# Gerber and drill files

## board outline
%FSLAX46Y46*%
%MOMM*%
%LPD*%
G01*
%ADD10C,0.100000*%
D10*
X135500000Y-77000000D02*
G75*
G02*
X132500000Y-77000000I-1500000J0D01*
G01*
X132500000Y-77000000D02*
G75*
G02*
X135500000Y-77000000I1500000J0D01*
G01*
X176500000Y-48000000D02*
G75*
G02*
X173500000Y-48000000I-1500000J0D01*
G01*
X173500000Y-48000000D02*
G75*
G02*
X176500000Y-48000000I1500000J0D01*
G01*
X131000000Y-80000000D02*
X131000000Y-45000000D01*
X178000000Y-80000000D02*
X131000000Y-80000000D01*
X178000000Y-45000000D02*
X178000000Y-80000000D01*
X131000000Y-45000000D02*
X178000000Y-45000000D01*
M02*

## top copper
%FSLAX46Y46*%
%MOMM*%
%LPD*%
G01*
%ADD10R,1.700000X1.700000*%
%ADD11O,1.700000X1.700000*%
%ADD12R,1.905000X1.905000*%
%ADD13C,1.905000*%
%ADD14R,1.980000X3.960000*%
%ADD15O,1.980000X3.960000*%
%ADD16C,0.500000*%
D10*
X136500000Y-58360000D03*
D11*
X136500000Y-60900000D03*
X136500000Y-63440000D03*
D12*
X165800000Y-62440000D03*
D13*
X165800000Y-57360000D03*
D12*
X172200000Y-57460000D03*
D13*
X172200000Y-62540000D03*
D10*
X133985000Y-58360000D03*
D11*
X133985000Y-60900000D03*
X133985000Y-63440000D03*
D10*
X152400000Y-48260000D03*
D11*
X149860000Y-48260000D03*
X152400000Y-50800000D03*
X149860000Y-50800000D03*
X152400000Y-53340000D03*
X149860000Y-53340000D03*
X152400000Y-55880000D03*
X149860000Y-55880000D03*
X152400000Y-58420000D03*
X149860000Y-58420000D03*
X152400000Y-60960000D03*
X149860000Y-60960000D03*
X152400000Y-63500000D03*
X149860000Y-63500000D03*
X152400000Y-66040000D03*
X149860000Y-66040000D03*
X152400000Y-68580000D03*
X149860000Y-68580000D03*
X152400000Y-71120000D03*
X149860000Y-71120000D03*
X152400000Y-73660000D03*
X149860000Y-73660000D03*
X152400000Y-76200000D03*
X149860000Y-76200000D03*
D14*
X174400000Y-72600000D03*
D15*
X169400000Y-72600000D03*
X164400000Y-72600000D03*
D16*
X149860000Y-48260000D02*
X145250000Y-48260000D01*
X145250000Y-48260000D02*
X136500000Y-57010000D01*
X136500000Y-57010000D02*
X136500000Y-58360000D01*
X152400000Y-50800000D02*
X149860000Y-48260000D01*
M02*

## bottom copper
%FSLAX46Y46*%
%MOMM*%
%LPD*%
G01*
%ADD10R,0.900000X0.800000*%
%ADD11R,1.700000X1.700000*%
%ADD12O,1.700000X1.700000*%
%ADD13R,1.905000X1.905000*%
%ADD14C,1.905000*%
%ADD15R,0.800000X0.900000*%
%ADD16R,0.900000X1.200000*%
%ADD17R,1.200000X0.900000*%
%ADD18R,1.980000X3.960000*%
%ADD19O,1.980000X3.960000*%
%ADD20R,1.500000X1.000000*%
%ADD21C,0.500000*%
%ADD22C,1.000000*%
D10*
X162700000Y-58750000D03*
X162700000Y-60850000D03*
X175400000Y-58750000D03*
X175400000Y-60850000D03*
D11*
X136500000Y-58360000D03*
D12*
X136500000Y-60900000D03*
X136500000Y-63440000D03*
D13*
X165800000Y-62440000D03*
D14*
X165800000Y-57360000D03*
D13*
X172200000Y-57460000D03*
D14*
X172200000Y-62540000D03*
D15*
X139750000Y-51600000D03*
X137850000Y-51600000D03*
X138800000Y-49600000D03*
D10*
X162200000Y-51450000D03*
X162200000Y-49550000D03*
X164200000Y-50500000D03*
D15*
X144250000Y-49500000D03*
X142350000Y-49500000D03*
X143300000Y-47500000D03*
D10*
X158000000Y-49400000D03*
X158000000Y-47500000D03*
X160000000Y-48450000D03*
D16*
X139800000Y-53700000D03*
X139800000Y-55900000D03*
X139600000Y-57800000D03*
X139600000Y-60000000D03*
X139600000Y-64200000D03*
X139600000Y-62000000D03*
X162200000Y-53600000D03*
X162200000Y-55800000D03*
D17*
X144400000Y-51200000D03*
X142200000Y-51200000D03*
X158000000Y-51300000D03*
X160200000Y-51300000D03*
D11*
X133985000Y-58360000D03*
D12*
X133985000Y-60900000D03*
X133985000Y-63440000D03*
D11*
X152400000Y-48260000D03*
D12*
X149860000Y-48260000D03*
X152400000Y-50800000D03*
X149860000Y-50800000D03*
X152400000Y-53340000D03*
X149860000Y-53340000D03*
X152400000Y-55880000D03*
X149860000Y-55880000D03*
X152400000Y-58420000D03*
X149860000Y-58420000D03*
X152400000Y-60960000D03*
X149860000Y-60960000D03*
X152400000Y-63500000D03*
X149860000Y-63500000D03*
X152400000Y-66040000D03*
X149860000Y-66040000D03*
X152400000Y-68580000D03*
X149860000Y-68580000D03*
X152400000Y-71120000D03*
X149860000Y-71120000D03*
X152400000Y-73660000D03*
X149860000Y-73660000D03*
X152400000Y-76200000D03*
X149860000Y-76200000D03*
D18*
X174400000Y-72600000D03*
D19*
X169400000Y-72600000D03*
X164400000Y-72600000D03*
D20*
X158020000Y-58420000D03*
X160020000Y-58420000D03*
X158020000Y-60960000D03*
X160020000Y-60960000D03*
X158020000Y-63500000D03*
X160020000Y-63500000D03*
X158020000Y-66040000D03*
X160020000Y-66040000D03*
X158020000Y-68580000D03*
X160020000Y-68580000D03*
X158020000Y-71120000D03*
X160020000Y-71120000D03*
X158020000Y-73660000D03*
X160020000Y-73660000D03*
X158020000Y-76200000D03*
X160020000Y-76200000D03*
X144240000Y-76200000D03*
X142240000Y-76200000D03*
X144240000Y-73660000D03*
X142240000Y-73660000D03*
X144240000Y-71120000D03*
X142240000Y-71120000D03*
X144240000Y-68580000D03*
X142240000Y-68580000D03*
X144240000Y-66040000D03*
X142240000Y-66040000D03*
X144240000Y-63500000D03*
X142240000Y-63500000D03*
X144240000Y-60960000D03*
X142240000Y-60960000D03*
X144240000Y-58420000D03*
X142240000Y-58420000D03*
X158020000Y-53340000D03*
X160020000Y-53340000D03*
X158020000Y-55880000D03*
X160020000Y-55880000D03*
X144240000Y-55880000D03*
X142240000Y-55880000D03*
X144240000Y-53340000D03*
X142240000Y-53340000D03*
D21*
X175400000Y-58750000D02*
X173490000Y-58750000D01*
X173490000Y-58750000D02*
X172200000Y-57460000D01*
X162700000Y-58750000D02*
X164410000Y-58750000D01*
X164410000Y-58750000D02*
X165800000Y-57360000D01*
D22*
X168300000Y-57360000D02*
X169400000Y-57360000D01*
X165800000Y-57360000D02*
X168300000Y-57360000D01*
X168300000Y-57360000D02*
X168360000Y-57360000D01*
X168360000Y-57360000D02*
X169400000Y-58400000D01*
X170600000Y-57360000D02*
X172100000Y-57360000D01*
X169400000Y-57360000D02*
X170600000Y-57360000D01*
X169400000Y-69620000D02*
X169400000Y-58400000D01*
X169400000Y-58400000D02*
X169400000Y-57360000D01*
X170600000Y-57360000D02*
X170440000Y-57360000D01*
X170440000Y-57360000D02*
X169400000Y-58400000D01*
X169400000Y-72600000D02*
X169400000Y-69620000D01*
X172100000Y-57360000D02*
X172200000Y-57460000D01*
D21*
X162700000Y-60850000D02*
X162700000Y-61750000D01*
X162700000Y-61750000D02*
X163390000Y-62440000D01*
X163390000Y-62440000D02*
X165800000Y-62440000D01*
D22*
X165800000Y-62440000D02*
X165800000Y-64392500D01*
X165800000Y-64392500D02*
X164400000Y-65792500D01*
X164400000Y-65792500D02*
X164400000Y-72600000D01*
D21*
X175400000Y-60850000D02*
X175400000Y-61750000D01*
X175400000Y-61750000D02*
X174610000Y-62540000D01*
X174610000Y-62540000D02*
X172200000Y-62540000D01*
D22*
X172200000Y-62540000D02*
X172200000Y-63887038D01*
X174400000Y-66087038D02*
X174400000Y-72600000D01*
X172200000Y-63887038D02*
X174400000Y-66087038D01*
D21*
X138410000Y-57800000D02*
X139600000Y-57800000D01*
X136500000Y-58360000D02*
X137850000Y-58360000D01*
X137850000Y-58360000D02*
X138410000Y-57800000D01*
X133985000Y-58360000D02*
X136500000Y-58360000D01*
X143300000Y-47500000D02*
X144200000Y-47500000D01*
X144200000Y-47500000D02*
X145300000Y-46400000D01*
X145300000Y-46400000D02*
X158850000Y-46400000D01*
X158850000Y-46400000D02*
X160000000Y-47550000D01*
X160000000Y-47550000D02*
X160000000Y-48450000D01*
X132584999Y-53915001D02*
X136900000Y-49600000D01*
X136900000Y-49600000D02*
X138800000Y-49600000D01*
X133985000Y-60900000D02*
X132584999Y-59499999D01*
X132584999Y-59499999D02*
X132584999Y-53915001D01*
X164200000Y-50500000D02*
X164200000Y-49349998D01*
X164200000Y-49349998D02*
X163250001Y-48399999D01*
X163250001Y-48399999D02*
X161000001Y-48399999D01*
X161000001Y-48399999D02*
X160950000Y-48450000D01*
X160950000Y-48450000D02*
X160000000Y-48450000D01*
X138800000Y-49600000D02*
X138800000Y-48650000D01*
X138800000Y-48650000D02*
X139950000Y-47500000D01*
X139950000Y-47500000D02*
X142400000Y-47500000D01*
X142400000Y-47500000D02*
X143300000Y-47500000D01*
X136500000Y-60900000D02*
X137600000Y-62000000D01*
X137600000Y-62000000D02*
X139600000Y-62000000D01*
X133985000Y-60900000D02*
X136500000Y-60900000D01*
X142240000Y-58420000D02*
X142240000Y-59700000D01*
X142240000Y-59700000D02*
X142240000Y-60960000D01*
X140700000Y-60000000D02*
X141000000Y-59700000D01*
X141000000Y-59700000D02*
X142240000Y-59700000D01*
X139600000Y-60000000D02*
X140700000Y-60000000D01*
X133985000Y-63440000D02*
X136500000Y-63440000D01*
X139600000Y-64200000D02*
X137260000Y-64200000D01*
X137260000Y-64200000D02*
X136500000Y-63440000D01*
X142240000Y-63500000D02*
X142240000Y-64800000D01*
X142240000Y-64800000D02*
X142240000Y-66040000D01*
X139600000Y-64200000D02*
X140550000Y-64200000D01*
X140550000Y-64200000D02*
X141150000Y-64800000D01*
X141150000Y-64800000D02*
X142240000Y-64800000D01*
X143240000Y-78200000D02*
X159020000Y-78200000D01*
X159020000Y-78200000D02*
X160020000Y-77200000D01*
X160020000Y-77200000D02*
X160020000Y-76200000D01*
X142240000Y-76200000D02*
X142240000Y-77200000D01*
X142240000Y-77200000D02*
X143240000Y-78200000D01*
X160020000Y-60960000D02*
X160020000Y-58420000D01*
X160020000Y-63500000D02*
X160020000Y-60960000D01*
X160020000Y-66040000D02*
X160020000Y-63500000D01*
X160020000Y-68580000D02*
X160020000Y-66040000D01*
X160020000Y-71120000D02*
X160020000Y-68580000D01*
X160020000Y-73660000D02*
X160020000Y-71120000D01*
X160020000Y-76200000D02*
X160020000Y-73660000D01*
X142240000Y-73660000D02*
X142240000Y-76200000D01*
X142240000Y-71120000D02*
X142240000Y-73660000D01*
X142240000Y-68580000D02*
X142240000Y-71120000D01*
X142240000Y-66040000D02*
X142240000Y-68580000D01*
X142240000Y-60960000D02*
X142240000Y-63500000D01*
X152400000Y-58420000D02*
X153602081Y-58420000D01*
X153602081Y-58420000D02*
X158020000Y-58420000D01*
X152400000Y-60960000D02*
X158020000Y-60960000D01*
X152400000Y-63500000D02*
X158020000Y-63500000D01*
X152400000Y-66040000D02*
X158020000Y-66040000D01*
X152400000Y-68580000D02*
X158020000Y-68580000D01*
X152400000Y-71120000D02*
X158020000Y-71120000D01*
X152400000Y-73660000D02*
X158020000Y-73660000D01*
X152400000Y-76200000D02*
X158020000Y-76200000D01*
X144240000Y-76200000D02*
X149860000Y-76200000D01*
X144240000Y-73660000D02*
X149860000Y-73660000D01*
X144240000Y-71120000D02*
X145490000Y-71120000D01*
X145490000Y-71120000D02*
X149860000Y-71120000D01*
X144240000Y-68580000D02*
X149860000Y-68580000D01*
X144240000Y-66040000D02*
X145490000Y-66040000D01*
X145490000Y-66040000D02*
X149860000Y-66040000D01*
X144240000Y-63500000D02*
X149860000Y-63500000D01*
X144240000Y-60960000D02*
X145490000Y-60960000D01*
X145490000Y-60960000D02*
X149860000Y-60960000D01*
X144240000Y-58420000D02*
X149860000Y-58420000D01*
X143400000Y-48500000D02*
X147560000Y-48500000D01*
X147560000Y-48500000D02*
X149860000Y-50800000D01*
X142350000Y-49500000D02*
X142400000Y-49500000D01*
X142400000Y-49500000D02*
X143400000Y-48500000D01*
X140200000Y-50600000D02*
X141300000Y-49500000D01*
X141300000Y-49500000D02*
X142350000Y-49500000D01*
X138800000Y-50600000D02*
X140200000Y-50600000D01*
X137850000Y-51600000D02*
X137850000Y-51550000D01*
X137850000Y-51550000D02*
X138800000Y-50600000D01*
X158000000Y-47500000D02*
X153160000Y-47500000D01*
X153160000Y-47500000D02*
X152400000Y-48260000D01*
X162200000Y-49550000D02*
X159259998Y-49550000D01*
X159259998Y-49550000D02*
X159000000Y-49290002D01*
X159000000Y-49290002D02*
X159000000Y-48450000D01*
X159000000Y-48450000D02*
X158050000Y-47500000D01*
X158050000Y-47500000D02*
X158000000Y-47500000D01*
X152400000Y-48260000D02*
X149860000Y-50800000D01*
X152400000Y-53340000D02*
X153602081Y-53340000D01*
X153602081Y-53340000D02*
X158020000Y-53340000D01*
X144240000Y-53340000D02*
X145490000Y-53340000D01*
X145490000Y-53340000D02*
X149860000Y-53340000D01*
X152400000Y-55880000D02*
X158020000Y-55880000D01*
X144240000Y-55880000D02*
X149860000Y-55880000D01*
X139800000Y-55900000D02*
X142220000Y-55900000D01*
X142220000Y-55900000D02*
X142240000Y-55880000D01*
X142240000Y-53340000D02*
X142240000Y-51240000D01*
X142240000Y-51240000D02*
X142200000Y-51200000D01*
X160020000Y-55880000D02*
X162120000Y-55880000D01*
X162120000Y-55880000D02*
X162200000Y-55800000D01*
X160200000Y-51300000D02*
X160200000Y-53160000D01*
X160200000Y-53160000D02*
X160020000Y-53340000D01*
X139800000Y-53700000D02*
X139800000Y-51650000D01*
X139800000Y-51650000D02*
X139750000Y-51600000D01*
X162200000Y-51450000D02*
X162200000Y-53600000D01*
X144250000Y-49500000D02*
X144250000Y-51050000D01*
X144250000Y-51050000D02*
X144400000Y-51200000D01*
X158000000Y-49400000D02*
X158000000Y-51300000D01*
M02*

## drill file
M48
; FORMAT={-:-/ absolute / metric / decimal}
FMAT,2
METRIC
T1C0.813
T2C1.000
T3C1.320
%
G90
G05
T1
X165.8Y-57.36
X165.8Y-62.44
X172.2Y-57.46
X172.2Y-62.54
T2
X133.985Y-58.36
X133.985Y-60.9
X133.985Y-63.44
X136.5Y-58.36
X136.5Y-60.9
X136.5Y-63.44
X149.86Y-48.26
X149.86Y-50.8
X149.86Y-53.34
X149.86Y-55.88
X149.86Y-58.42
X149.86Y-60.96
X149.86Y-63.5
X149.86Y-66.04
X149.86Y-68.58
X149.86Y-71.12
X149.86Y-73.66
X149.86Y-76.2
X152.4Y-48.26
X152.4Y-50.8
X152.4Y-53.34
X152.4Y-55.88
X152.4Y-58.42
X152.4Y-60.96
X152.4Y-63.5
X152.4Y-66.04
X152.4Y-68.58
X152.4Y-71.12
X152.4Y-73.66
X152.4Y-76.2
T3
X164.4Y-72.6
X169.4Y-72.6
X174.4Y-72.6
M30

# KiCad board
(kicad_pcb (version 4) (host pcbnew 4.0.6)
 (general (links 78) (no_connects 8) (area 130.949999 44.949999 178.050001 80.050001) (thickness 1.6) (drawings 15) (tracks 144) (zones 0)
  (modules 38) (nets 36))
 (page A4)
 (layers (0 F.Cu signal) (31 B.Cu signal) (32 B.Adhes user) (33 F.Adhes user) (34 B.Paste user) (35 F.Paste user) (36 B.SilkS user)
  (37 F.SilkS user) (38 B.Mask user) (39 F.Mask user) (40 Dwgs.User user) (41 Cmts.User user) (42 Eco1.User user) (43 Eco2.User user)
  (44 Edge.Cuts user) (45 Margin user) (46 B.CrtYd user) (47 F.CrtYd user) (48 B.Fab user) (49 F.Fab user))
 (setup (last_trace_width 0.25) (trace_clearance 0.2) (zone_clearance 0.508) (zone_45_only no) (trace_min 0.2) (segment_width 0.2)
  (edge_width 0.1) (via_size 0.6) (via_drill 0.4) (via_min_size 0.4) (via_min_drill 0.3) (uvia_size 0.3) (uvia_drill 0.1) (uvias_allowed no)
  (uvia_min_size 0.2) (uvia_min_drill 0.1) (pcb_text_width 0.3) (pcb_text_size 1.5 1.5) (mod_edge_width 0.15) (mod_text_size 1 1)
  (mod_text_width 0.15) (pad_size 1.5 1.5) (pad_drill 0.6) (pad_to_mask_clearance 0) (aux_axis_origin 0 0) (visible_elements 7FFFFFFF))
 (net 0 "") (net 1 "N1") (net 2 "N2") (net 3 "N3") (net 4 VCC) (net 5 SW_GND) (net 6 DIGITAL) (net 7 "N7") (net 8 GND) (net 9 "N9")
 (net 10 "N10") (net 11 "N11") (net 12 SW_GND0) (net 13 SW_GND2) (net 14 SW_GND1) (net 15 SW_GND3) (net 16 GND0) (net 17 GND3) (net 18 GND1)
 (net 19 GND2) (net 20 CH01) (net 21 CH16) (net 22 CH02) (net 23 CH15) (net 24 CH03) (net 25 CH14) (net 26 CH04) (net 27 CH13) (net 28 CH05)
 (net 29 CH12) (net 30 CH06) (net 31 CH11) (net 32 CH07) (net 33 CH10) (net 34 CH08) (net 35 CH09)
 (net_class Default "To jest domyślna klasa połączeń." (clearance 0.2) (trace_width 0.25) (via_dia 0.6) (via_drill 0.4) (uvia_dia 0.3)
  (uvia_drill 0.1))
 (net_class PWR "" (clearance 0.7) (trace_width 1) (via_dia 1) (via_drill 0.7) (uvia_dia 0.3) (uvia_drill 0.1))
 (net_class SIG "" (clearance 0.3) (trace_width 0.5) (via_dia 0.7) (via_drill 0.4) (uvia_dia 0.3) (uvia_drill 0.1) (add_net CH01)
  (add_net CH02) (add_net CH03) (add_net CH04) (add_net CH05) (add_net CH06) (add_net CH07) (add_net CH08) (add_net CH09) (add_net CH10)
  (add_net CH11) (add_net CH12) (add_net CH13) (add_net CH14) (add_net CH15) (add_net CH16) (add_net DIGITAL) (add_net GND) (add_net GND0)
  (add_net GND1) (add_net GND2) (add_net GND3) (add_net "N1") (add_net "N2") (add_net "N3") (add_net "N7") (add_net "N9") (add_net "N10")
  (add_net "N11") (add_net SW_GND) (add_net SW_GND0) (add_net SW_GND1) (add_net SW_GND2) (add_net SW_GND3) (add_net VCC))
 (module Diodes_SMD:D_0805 (layer B.Cu) (at 162.7 59.8 270)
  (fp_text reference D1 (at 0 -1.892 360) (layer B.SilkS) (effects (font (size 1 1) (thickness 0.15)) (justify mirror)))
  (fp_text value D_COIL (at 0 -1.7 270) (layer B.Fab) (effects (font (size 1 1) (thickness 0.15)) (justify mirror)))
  (pad 1 smd rect (at -1.05 0 270) (size 0.8 0.9) (layers B.Cu B.Paste B.Mask) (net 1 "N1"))
  (pad 2 smd rect (at 1.05 0 270) (size 0.8 0.9) (layers B.Cu B.Paste B.Mask) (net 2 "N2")))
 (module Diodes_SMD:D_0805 (layer B.Cu) (at 175.4 59.8 270)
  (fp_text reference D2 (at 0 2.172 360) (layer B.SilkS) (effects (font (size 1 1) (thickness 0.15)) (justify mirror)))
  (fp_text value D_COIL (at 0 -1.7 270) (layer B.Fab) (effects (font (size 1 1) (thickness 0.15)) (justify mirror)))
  (pad 1 smd rect (at -1.05 0 270) (size 0.8 0.9) (layers B.Cu B.Paste B.Mask) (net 1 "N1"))
  (pad 2 smd rect (at 1.05 0 270) (size 0.8 0.9) (layers B.Cu B.Paste B.Mask) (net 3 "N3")))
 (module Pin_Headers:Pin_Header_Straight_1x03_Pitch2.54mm (layer F.Cu) (at 136.5 58.36)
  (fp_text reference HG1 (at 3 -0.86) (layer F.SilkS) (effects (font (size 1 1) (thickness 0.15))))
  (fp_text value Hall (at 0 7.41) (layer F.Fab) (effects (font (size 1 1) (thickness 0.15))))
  (pad 1 thru_hole rect (at 0 0) (size 1.7 1.7) (drill 1) (layers *.Cu *.Mask) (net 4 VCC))
  (pad 2 thru_hole oval (at 0 2.54) (size 1.7 1.7) (drill 1) (layers *.Cu *.Mask) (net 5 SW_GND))
  (pad 3 thru_hole oval (at 0 5.08) (size 1.7 1.7) (drill 1) (layers *.Cu *.Mask) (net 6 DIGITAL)))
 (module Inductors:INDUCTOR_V (layer F.Cu) (at 165.8 59.9 90)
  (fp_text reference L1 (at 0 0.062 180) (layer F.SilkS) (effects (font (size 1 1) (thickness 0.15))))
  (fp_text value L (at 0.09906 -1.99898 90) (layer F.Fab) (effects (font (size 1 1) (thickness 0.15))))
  (pad 1 thru_hole rect (at -2.54 0 90) (size 1.905 1.905) (drill 0.8128) (layers *.Cu *.Mask) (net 2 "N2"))
  (pad 2 thru_hole circle (at 2.54 0 90) (size 1.905 1.905) (drill 0.8128) (layers *.Cu *.Mask) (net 1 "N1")))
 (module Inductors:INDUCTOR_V (layer F.Cu) (at 172.2 60 270)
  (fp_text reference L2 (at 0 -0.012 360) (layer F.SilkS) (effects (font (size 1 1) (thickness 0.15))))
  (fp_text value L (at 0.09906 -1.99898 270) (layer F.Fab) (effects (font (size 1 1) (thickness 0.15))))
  (pad 1 thru_hole rect (at -2.54 0 270) (size 1.905 1.905) (drill 0.8128) (layers *.Cu *.Mask) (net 1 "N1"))
  (pad 2 thru_hole circle (at 2.54 0 270) (size 1.905 1.905) (drill 0.8128) (layers *.Cu *.Mask) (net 3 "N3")))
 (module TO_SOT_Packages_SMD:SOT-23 (layer B.Cu) (at 138.8 50.6 90)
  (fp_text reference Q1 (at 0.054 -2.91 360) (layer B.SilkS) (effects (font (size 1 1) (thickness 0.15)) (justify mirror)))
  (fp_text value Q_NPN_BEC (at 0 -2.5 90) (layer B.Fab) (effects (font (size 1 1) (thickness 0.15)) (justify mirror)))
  (pad 1 smd rect (at -1 0.95 90) (size 0.9 0.8) (layers B.Cu B.Paste B.Mask) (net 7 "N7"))
  (pad 2 smd rect (at -1 -0.95 90) (size 0.9 0.8) (layers B.Cu B.Paste B.Mask) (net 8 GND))
  (pad 3 smd rect (at 1 0 90) (size 0.9 0.8) (layers B.Cu B.Paste B.Mask) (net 5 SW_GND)))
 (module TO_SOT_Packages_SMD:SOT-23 (layer B.Cu) (at 163.2 50.5)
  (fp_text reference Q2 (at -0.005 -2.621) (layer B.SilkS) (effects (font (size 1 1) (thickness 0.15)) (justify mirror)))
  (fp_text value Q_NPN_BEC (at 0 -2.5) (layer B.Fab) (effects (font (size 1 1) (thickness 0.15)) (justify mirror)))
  (pad 1 smd rect (at -1 0.95) (size 0.9 0.8) (layers B.Cu B.Paste B.Mask) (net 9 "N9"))
  (pad 2 smd rect (at -1 -0.95) (size 0.9 0.8) (layers B.Cu B.Paste B.Mask) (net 8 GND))
  (pad 3 smd rect (at 1 0) (size 0.9 0.8) (layers B.Cu B.Paste B.Mask) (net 5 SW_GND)))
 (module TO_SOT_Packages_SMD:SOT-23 (layer B.Cu) (at 143.3 48.5 90)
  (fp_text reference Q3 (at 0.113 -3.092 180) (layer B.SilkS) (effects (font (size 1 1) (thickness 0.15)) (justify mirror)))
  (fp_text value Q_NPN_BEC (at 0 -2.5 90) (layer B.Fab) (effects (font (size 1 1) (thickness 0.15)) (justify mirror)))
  (pad 1 smd rect (at -1 0.95 90) (size 0.9 0.8) (layers B.Cu B.Paste B.Mask) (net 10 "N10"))
  (pad 2 smd rect (at -1 -0.95 90) (size 0.9 0.8) (layers B.Cu B.Paste B.Mask) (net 8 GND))
  (pad 3 smd rect (at 1 0 90) (size 0.9 0.8) (layers B.Cu B.Paste B.Mask) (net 5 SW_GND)))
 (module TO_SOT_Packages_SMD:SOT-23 (layer B.Cu) (at 159 48.45)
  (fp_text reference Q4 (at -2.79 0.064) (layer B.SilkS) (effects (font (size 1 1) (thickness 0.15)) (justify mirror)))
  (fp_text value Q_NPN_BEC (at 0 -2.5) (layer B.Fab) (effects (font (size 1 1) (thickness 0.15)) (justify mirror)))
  (pad 1 smd rect (at -1 0.95) (size 0.9 0.8) (layers B.Cu B.Paste B.Mask) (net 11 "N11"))
  (pad 2 smd rect (at -1 -0.95) (size 0.9 0.8) (layers B.Cu B.Paste B.Mask) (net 8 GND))
  (pad 3 smd rect (at 1 0) (size 0.9 0.8) (layers B.Cu B.Paste B.Mask) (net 5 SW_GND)))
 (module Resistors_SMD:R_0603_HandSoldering (layer B.Cu) (at 139.8 54.8 270)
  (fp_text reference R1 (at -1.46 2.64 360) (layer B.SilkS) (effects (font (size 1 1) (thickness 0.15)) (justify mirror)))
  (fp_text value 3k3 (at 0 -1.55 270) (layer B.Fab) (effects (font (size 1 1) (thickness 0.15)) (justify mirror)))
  (pad 1 smd rect (at -1.1 0 270) (size 1.2 0.9) (layers B.Cu B.Paste B.Mask) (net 7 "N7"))
  (pad 2 smd rect (at 1.1 0 270) (size 1.2 0.9) (layers B.Cu B.Paste B.Mask) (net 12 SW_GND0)))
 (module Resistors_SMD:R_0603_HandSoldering (layer B.Cu) (at 139.6 58.9 270)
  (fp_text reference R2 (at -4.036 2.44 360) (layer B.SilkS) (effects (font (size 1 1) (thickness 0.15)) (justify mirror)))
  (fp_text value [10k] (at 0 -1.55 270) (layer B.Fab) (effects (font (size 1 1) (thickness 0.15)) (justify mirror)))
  (pad 1 smd rect (at -1.1 0 270) (size 1.2 0.9) (layers B.Cu B.Paste B.Mask) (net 4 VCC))
  (pad 2 smd rect (at 1.1 0 270) (size 1.2 0.9) (layers B.Cu B.Paste B.Mask) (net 6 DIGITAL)))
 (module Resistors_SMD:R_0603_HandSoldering (layer B.Cu) (at 139.6 63.1 90)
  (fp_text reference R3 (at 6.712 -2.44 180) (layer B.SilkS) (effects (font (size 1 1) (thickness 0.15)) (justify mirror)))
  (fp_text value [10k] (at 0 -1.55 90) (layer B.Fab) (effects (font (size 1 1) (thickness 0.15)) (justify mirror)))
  (pad 1 smd rect (at -1.1 0 90) (size 1.2 0.9) (layers B.Cu B.Paste B.Mask) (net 6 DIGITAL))
  (pad 2 smd rect (at 1.1 0 90) (size 1.2 0.9) (layers B.Cu B.Paste B.Mask) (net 5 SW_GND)))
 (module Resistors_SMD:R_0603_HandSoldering (layer B.Cu) (at 162.2 54.7 270)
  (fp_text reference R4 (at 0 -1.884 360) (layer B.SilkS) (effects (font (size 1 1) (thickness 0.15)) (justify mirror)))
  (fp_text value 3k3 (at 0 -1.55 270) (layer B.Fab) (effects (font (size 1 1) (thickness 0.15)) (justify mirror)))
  (pad 1 smd rect (at -1.1 0 270) (size 1.2 0.9) (layers B.Cu B.Paste B.Mask) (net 9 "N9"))
  (pad 2 smd rect (at 1.1 0 270) (size 1.2 0.9) (layers B.Cu B.Paste B.Mask) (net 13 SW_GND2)))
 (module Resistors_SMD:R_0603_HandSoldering (layer B.Cu) (at 143.3 51.2 180)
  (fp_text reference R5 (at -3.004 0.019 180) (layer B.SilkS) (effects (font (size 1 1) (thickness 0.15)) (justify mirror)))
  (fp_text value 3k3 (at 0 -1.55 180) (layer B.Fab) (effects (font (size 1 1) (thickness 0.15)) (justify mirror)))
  (pad 1 smd rect (at -1.1 0 180) (size 1.2 0.9) (layers B.Cu B.Paste B.Mask) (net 10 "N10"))
  (pad 2 smd rect (at 1.1 0 180) (size 1.2 0.9) (layers B.Cu B.Paste B.Mask) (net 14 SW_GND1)))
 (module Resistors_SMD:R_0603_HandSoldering (layer B.Cu) (at 159.1 51.3)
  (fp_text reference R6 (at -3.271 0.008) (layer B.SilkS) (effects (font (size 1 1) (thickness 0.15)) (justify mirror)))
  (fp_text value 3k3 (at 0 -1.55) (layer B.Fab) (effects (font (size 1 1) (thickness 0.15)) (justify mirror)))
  (pad 1 smd rect (at -1.1 0) (size 1.2 0.9) (layers B.Cu B.Paste B.Mask) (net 11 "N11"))
  (pad 2 smd rect (at 1.1 0) (size 1.2 0.9) (layers B.Cu B.Paste B.Mask) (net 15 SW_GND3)))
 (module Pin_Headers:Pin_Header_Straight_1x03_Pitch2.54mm (layer F.Cu) (at 133.985 58.36)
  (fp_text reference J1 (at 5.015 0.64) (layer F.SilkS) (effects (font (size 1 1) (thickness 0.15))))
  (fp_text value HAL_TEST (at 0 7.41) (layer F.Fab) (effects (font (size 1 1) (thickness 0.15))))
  (pad 1 thru_hole rect (at 0 0) (size 1.7 1.7) (drill 1) (layers *.Cu *.Mask) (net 4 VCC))
  (pad 2 thru_hole oval (at 0 2.54) (size 1.7 1.7) (drill 1) (layers *.Cu *.Mask) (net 5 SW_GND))
  (pad 3 thru_hole oval (at 0 5.08) (size 1.7 1.7) (drill 1) (layers *.Cu *.Mask) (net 6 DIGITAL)))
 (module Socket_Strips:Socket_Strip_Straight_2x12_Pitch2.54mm (layer F.Cu) (at 152.4 48.26)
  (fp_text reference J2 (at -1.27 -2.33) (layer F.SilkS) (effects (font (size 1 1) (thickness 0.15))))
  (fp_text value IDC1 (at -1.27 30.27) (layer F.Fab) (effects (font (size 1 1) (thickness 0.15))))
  (pad 1 thru_hole rect (at 0 0) (size 1.7 1.7) (drill 1) (layers *.Cu *.Mask) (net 8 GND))
  (pad 2 thru_hole oval (at -2.54 0) (size 1.7 1.7) (drill 1) (layers *.Cu *.Mask) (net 4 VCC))
  (pad 3 thru_hole oval (at 0 2.54) (size 1.7 1.7) (drill 1) (layers *.Cu *.Mask) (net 4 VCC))
  (pad 4 thru_hole oval (at -2.54 2.54) (size 1.7 1.7) (drill 1) (layers *.Cu *.Mask) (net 8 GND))
  (pad 5 thru_hole oval (at 0 5.08) (size 1.7 1.7) (drill 1) (layers *.Cu *.Mask) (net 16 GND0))
  (pad 6 thru_hole oval (at -2.54 5.08) (size 1.7 1.7) (drill 1) (layers *.Cu *.Mask) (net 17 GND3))
  (pad 7 thru_hole oval (at 0 7.62) (size 1.7 1.7) (drill 1) (layers *.Cu *.Mask) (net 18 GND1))
  (pad 8 thru_hole oval (at -2.54 7.62) (size 1.7 1.7) (drill 1) (layers *.Cu *.Mask) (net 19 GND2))
  (pad 9 thru_hole oval (at 0 10.16) (size 1.7 1.7) (drill 1) (layers *.Cu *.Mask) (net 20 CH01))
  (pad 10 thru_hole oval (at -2.54 10.16) (size 1.7 1.7) (drill 1) (layers *.Cu *.Mask) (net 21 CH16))
  (pad 11 thru_hole oval (at 0 12.7) (size 1.7 1.7) (drill 1) (layers *.Cu *.Mask) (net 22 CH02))
  (pad 12 thru_hole oval (at -2.54 12.7) (size 1.7 1.7) (drill 1) (layers *.Cu *.Mask) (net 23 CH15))
  (pad 13 thru_hole oval (at 0 15.24) (size 1.7 1.7) (drill 1) (layers *.Cu *.Mask) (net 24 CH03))
  (pad 14 thru_hole oval (at -2.54 15.24) (size 1.7 1.7) (drill 1) (layers *.Cu *.Mask) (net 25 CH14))
  (pad 15 thru_hole oval (at 0 17.78) (size 1.7 1.7) (drill 1) (layers *.Cu *.Mask) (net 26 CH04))
  (pad 16 thru_hole oval (at -2.54 17.78) (size 1.7 1.7) (drill 1) (layers *.Cu *.Mask) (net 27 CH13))
  (pad 17 thru_hole oval (at 0 20.32) (size 1.7 1.7) (drill 1) (layers *.Cu *.Mask) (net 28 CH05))
  (pad 18 thru_hole oval (at -2.54 20.32) (size 1.7 1.7) (drill 1) (layers *.Cu *.Mask) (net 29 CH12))
  (pad 19 thru_hole oval (at 0 22.86) (size 1.7 1.7) (drill 1) (layers *.Cu *.Mask) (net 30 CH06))
  (pad 20 thru_hole oval (at -2.54 22.86) (size 1.7 1.7) (drill 1) (layers *.Cu *.Mask) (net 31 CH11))
  (pad 21 thru_hole oval (at 0 25.4) (size 1.7 1.7) (drill 1) (layers *.Cu *.Mask) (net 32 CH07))
  (pad 22 thru_hole oval (at -2.54 25.4) (size 1.7 1.7) (drill 1) (layers *.Cu *.Mask) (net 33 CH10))
  (pad 23 thru_hole oval (at 0 27.94) (size 1.7 1.7) (drill 1) (layers *.Cu *.Mask) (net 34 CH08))
  (pad 24 thru_hole oval (at -2.54 27.94) (size 1.7 1.7) (drill 1) (layers *.Cu *.Mask) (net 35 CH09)))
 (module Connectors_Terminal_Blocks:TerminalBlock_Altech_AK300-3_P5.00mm (layer F.Cu) (at 174.4 72.6 180)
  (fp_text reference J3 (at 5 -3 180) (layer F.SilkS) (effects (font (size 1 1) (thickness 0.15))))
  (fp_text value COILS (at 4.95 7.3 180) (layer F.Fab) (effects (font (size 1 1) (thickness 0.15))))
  (pad 1 thru_hole rect (at 0 0 180) (size 1.98 3.96) (drill 1.32) (layers *.Cu *.Mask) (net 3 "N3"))
  (pad 2 thru_hole oval (at 5 0 180) (size 1.98 3.96) (drill 1.32) (layers *.Cu *.Mask) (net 1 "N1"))
  (pad 3 thru_hole oval (at 10 0 180) (size 1.98 3.96) (drill 1.32) (layers *.Cu *.Mask) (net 2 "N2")))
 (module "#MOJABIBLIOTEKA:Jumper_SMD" (layer B.Cu) (at 159.02 58.42)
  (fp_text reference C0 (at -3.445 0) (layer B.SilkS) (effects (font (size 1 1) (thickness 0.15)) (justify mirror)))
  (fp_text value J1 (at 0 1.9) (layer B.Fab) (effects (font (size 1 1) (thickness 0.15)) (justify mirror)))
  (pad 1 smd rect (at -1 0) (size 1.5 1) (layers B.Cu B.Paste B.Mask) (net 20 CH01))
  (pad 2 smd rect (at 1 0) (size 1.5 1) (layers B.Cu B.Paste B.Mask) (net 6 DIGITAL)))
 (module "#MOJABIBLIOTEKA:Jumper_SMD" (layer B.Cu) (at 159.02 60.96)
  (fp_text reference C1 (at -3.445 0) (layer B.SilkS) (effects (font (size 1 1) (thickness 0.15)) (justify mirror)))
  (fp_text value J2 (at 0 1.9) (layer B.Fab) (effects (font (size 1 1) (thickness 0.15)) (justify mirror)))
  (pad 1 smd rect (at -1 0) (size 1.5 1) (layers B.Cu B.Paste B.Mask) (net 22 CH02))
  (pad 2 smd rect (at 1 0) (size 1.5 1) (layers B.Cu B.Paste B.Mask) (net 6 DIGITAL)))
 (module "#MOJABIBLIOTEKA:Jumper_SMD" (layer B.Cu) (at 159.02 63.5)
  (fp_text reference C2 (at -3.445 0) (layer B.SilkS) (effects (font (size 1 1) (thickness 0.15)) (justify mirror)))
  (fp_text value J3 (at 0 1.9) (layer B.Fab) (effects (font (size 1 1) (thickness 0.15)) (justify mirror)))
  (pad 1 smd rect (at -1 0) (size 1.5 1) (layers B.Cu B.Paste B.Mask) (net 24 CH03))
  (pad 2 smd rect (at 1 0) (size 1.5 1) (layers B.Cu B.Paste B.Mask) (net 6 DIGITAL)))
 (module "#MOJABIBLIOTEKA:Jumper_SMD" (layer B.Cu) (at 159.02 66.04)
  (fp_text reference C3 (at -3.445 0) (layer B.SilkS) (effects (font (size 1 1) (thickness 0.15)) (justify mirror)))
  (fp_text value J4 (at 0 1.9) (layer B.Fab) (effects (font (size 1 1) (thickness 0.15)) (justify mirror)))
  (pad 1 smd rect (at -1 0) (size 1.5 1) (layers B.Cu B.Paste B.Mask) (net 26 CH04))
  (pad 2 smd rect (at 1 0) (size 1.5 1) (layers B.Cu B.Paste B.Mask) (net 6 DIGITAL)))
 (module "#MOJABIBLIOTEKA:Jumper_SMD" (layer B.Cu) (at 159.02 68.58)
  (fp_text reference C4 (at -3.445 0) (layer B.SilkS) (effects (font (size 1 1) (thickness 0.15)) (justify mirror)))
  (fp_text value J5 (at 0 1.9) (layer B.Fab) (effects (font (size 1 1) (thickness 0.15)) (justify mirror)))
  (pad 1 smd rect (at -1 0) (size 1.5 1) (layers B.Cu B.Paste B.Mask) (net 28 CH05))
  (pad 2 smd rect (at 1 0) (size 1.5 1) (layers B.Cu B.Paste B.Mask) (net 6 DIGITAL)))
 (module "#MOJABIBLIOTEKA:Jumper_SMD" (layer B.Cu) (at 159.02 71.12)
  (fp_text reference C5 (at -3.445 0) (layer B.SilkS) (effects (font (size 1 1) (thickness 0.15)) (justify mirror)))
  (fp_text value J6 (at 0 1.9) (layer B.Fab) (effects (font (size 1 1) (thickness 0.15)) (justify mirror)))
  (pad 1 smd rect (at -1 0) (size 1.5 1) (layers B.Cu B.Paste B.Mask) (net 30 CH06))
  (pad 2 smd rect (at 1 0) (size 1.5 1) (layers B.Cu B.Paste B.Mask) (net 6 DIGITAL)))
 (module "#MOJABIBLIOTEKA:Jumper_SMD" (layer B.Cu) (at 159.02 73.66)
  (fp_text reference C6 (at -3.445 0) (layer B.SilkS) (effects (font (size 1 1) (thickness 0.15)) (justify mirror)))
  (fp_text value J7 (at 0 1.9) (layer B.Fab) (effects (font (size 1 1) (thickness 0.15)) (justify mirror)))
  (pad 1 smd rect (at -1 0) (size 1.5 1) (layers B.Cu B.Paste B.Mask) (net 32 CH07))
  (pad 2 smd rect (at 1 0) (size 1.5 1) (layers B.Cu B.Paste B.Mask) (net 6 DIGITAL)))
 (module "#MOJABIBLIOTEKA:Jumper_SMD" (layer B.Cu) (at 159.02 76.2)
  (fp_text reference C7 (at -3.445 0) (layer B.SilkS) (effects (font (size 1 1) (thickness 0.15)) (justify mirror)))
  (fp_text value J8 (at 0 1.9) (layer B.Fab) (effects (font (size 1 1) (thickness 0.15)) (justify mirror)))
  (pad 1 smd rect (at -1 0) (size 1.5 1) (layers B.Cu B.Paste B.Mask) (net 34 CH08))
  (pad 2 smd rect (at 1 0) (size 1.5 1) (layers B.Cu B.Paste B.Mask) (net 6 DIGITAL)))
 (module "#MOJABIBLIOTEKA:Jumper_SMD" (layer B.Cu) (at 143.24 76.2 180)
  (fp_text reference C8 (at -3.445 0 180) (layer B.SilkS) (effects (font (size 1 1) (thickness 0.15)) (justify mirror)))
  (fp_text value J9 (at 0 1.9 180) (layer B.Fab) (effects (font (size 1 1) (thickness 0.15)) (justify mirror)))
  (pad 1 smd rect (at -1 0 180) (size 1.5 1) (layers B.Cu B.Paste B.Mask) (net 35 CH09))
  (pad 2 smd rect (at 1 0 180) (size 1.5 1) (layers B.Cu B.Paste B.Mask) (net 6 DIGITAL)))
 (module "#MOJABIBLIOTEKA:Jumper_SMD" (layer B.Cu) (at 143.24 73.66 180)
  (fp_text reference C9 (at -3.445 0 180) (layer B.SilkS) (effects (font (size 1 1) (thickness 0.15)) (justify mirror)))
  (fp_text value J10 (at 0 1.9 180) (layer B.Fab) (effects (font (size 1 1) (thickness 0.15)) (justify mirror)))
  (pad 1 smd rect (at -1 0 180) (size 1.5 1) (layers B.Cu B.Paste B.Mask) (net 33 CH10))
  (pad 2 smd rect (at 1 0 180) (size 1.5 1) (layers B.Cu B.Paste B.Mask) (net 6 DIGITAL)))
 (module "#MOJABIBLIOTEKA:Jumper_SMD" (layer B.Cu) (at 143.24 71.12 180)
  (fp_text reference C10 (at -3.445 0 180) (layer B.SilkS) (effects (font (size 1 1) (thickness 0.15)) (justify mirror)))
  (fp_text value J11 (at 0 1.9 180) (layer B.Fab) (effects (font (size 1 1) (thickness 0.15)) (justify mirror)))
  (pad 1 smd rect (at -1 0 180) (size 1.5 1) (layers B.Cu B.Paste B.Mask) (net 31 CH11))
  (pad 2 smd rect (at 1 0 180) (size 1.5 1) (layers B.Cu B.Paste B.Mask) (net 6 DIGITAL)))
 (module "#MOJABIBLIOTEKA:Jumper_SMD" (layer B.Cu) (at 143.24 68.58 180)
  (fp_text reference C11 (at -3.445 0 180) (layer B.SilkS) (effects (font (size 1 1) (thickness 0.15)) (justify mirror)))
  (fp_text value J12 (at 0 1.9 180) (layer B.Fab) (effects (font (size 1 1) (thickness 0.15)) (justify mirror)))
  (pad 1 smd rect (at -1 0 180) (size 1.5 1) (layers B.Cu B.Paste B.Mask) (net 29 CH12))
  (pad 2 smd rect (at 1 0 180) (size 1.5 1) (layers B.Cu B.Paste B.Mask) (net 6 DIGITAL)))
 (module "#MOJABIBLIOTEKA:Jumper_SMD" (layer B.Cu) (at 143.24 66.04 180)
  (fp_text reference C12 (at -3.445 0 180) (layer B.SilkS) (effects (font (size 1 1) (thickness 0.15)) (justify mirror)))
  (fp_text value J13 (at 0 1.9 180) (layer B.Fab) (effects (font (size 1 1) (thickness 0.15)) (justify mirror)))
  (pad 1 smd rect (at -1 0 180) (size 1.5 1) (layers B.Cu B.Paste B.Mask) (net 27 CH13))
  (pad 2 smd rect (at 1 0 180) (size 1.5 1) (layers B.Cu B.Paste B.Mask) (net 6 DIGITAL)))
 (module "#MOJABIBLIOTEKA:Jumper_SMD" (layer B.Cu) (at 143.24 63.5 180)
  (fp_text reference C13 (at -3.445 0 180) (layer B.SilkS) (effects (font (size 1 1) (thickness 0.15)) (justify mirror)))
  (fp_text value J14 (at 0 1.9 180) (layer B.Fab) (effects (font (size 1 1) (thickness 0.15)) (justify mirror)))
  (pad 1 smd rect (at -1 0 180) (size 1.5 1) (layers B.Cu B.Paste B.Mask) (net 25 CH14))
  (pad 2 smd rect (at 1 0 180) (size 1.5 1) (layers B.Cu B.Paste B.Mask) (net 6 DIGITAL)))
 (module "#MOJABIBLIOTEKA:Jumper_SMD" (layer B.Cu) (at 143.24 60.96 180)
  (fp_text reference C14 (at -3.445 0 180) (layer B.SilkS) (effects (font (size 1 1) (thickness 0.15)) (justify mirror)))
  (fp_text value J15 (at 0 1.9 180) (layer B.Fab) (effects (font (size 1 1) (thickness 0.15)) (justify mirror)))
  (pad 1 smd rect (at -1 0 180) (size 1.5 1) (layers B.Cu B.Paste B.Mask) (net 23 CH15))
  (pad 2 smd rect (at 1 0 180) (size 1.5 1) (layers B.Cu B.Paste B.Mask) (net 6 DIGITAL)))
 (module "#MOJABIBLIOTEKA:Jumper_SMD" (layer B.Cu) (at 143.24 58.42 180)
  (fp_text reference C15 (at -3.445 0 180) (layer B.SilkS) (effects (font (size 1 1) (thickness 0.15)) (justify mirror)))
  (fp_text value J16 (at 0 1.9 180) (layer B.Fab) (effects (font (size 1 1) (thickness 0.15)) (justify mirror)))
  (pad 1 smd rect (at -1 0 180) (size 1.5 1) (layers B.Cu B.Paste B.Mask) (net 21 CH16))
  (pad 2 smd rect (at 1 0 180) (size 1.5 1) (layers B.Cu B.Paste B.Mask) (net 6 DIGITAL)))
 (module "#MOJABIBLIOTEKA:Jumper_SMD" (layer B.Cu) (at 159.02 53.34)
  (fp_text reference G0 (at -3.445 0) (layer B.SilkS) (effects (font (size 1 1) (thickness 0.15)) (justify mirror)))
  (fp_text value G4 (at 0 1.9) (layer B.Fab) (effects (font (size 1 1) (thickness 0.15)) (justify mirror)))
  (pad 1 smd rect (at -1 0) (size 1.5 1) (layers B.Cu B.Paste B.Mask) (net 16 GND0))
  (pad 2 smd rect (at 1 0) (size 1.5 1) (layers B.Cu B.Paste B.Mask) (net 15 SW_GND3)))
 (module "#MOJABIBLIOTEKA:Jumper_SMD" (layer B.Cu) (at 159.02 55.88)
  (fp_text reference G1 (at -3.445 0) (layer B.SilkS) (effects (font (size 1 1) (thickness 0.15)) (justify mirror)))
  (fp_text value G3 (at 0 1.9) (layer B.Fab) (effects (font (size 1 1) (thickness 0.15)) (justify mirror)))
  (pad 1 smd rect (at -1 0) (size 1.5 1) (layers B.Cu B.Paste B.Mask) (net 18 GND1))
  (pad 2 smd rect (at 1 0) (size 1.5 1) (layers B.Cu B.Paste B.Mask) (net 13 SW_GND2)))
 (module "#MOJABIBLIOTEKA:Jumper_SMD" (layer B.Cu) (at 143.24 55.88 180)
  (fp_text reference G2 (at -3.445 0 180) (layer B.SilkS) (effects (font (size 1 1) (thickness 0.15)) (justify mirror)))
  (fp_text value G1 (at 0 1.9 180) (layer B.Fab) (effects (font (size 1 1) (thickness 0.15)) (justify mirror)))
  (pad 1 smd rect (at -1 0 180) (size 1.5 1) (layers B.Cu B.Paste B.Mask) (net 19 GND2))
  (pad 2 smd rect (at 1 0 180) (size 1.5 1) (layers B.Cu B.Paste B.Mask) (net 12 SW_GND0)))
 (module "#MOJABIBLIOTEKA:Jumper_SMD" (layer B.Cu) (at 143.24 53.34 180)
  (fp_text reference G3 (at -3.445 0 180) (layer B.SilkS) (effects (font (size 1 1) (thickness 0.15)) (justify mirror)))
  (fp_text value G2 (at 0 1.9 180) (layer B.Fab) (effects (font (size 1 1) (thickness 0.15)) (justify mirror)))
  (pad 1 smd rect (at -1 0 180) (size 1.5 1) (layers B.Cu B.Paste B.Mask) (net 17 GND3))
  (pad 2 smd rect (at 1 0 180) (size 1.5 1) (layers B.Cu B.Paste B.Mask) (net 14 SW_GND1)))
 (gr_circle (center 134 77) (end 134 78.5) (layer Edge.Cuts) (width 0.1))
 (gr_circle (center 175 48) (end 175 46.5) (layer Edge.Cuts) (width 0.1))
 (gr_line (start 131 80) (end 131 45) (layer Edge.Cuts) (width 0.1))
 (gr_line (start 178 80) (end 131 80) (layer Edge.Cuts) (width 0.1))
 (gr_line (start 178 45) (end 178 80) (layer Edge.Cuts) (width 0.1))
 (gr_line (start 131 45) (end 178 45) (layer Edge.Cuts) (width 0.1))
 (segment (start 175.4 58.75) (end 173.49 58.75) (width 0.5) (layer B.Cu) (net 1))
 (segment (start 173.49 58.75) (end 172.2 57.46) (width 0.5) (layer B.Cu) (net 1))
 (segment (start 162.7 58.75) (end 164.41 58.75) (width 0.5) (layer B.Cu) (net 1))
 (segment (start 164.41 58.75) (end 165.8 57.36) (width 0.5) (layer B.Cu) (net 1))
 (segment (start 168.3 57.36) (end 169.4 57.36) (width 1) (layer B.Cu) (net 1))
 (segment (start 165.8 57.36) (end 168.3 57.36) (width 1) (layer B.Cu) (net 1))
 (segment (start 168.3 57.36) (end 168.36 57.36) (width 1) (layer B.Cu) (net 1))
 (segment (start 168.36 57.36) (end 169.4 58.4) (width 1) (layer B.Cu) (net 1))
 (segment (start 170.6 57.36) (end 172.1 57.36) (width 1) (layer B.Cu) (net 1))
 (segment (start 169.4 57.36) (end 170.6 57.36) (width 1) (layer B.Cu) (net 1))
 (segment (start 169.4 69.62) (end 169.4 58.4) (width 1) (layer B.Cu) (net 1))
 (segment (start 169.4 58.4) (end 169.4 57.36) (width 1) (layer B.Cu) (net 1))
 (segment (start 170.6 57.36) (end 170.44 57.36) (width 1) (layer B.Cu) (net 1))
 (segment (start 170.44 57.36) (end 169.4 58.4) (width 1) (layer B.Cu) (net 1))
 (segment (start 169.4 72.6) (end 169.4 69.62) (width 1) (layer B.Cu) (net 1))
 (segment (start 172.1 57.36) (end 172.2 57.46) (width 1) (layer B.Cu) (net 1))
 (segment (start 162.7 60.85) (end 162.7 61.75) (width 0.5) (layer B.Cu) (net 2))
 (segment (start 162.7 61.75) (end 163.39 62.44) (width 0.5) (layer B.Cu) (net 2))
 (segment (start 163.39 62.44) (end 165.8 62.44) (width 0.5) (layer B.Cu) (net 2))
 (segment (start 165.8 62.44) (end 165.8 64.3925) (width 1) (layer B.Cu) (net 2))
 (segment (start 165.8 64.3925) (end 164.4 65.7925) (width 1) (layer B.Cu) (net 2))
 (segment (start 164.4 65.7925) (end 164.4 72.6) (width 1) (layer B.Cu) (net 2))
 (segment (start 175.4 60.85) (end 175.4 61.75) (width 0.5) (layer B.Cu) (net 3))
 (segment (start 175.4 61.75) (end 174.61 62.54) (width 0.5) (layer B.Cu) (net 3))
 (segment (start 174.61 62.54) (end 172.2 62.54) (width 0.5) (layer B.Cu) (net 3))
 (segment (start 172.2 62.54) (end 172.2 63.887038) (width 1) (layer B.Cu) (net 3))
 (segment (start 174.4 66.087038) (end 174.4 72.6) (width 1) (layer B.Cu) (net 3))
 (segment (start 172.2 63.887038) (end 174.4 66.087038) (width 1) (layer B.Cu) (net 3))
 (segment (start 149.86 48.26) (end 145.25 48.26) (width 0.5) (layer F.Cu) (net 4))
 (segment (start 145.25 48.26) (end 136.5 57.01) (width 0.5) (layer F.Cu) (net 4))
 (segment (start 136.5 57.01) (end 136.5 58.36) (width 0.5) (layer F.Cu) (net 4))
 (segment (start 152.4 50.8) (end 149.86 48.26) (width 0.5) (layer F.Cu) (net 4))
 (segment (start 138.41 57.8) (end 139.6 57.8) (width 0.5) (layer B.Cu) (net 4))
 (segment (start 136.5 58.36) (end 137.85 58.36) (width 0.5) (layer B.Cu) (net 4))
 (segment (start 137.85 58.36) (end 138.41 57.8) (width 0.5) (layer B.Cu) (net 4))
 (segment (start 133.985 58.36) (end 136.5 58.36) (width 0.5) (layer B.Cu) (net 4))
 (segment (start 143.3 47.5) (end 144.2 47.5) (width 0.5) (layer B.Cu) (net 5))
 (segment (start 144.2 47.5) (end 145.3 46.4) (width 0.5) (layer B.Cu) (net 5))
 (segment (start 145.3 46.4) (end 158.85 46.4) (width 0.5) (layer B.Cu) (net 5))
 (segment (start 158.85 46.4) (end 160 47.55) (width 0.5) (layer B.Cu) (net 5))
 (segment (start 160 47.55) (end 160 48.45) (width 0.5) (layer B.Cu) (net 5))
 (segment (start 132.584999 53.915001) (end 136.9 49.6) (width 0.5) (layer B.Cu) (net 5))
 (segment (start 136.9 49.6) (end 138.8 49.6) (width 0.5) (layer B.Cu) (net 5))
 (segment (start 133.985 60.9) (end 132.584999 59.499999) (width 0.5) (layer B.Cu) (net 5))
 (segment (start 132.584999 59.499999) (end 132.584999 53.915001) (width 0.5) (layer B.Cu) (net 5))
 (segment (start 164.2 50.5) (end 164.2 49.349998) (width 0.5) (layer B.Cu) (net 5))
 (segment (start 164.2 49.349998) (end 163.250001 48.399999) (width 0.5) (layer B.Cu) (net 5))
 (segment (start 163.250001 48.399999) (end 161.000001 48.399999) (width 0.5) (layer B.Cu) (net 5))
 (segment (start 161.000001 48.399999) (end 160.95 48.45) (width 0.5) (layer B.Cu) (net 5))
 (segment (start 160.95 48.45) (end 160 48.45) (width 0.5) (layer B.Cu) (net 5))
 (segment (start 138.8 49.6) (end 138.8 48.65) (width 0.5) (layer B.Cu) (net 5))
 (segment (start 138.8 48.65) (end 139.95 47.5) (width 0.5) (layer B.Cu) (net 5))
 (segment (start 139.95 47.5) (end 142.4 47.5) (width 0.5) (layer B.Cu) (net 5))
 (segment (start 142.4 47.5) (end 143.3 47.5) (width 0.5) (layer B.Cu) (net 5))
 (segment (start 136.5 60.9) (end 137.6 62) (width 0.5) (layer B.Cu) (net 5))
 (segment (start 137.6 62) (end 139.6 62) (width 0.5) (layer B.Cu) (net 5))
 (segment (start 133.985 60.9) (end 136.5 60.9) (width 0.5) (layer B.Cu) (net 5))
 (segment (start 142.24 58.42) (end 142.24 59.7) (width 0.5) (layer B.Cu) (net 6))
 (segment (start 142.24 59.7) (end 142.24 60.96) (width 0.5) (layer B.Cu) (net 6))
 (segment (start 140.7 60) (end 141 59.7) (width 0.5) (layer B.Cu) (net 6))
 (segment (start 141 59.7) (end 142.24 59.7) (width 0.5) (layer B.Cu) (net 6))
 (segment (start 139.6 60) (end 140.7 60) (width 0.5) (layer B.Cu) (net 6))
 (segment (start 133.985 63.44) (end 136.5 63.44) (width 0.5) (layer B.Cu) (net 6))
 (segment (start 139.6 64.2) (end 137.26 64.2) (width 0.5) (layer B.Cu) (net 6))
 (segment (start 137.26 64.2) (end 136.5 63.44) (width 0.5) (layer B.Cu) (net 6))
 (segment (start 142.24 63.5) (end 142.24 64.8) (width 0.5) (layer B.Cu) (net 6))
 (segment (start 142.24 64.8) (end 142.24 66.04) (width 0.5) (layer B.Cu) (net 6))
 (segment (start 139.6 64.2) (end 140.55 64.2) (width 0.5) (layer B.Cu) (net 6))
 (segment (start 140.55 64.2) (end 141.15 64.8) (width 0.5) (layer B.Cu) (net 6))
 (segment (start 141.15 64.8) (end 142.24 64.8) (width 0.5) (layer B.Cu) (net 6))
 (segment (start 143.24 78.2) (end 159.02 78.2) (width 0.5) (layer B.Cu) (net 6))
 (segment (start 159.02 78.2) (end 160.02 77.2) (width 0.5) (layer B.Cu) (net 6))
 (segment (start 160.02 77.2) (end 160.02 76.2) (width 0.5) (layer B.Cu) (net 6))
 (segment (start 142.24 76.2) (end 142.24 77.2) (width 0.5) (layer B.Cu) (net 6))
 (segment (start 142.24 77.2) (end 143.24 78.2) (width 0.5) (layer B.Cu) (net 6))
 (segment (start 160.02 60.96) (end 160.02 58.42) (width 0.5) (layer B.Cu) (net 6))
 (segment (start 160.02 63.5) (end 160.02 60.96) (width 0.5) (layer B.Cu) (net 6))
 (segment (start 160.02 66.04) (end 160.02 63.5) (width 0.5) (layer B.Cu) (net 6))
 (segment (start 160.02 68.58) (end 160.02 66.04) (width 0.5) (layer B.Cu) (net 6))
 (segment (start 160.02 71.12) (end 160.02 68.58) (width 0.5) (layer B.Cu) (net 6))
 (segment (start 160.02 73.66) (end 160.02 71.12) (width 0.5) (layer B.Cu) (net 6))
 (segment (start 160.02 76.2) (end 160.02 73.66) (width 0.5) (layer B.Cu) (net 6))
 (segment (start 142.24 73.66) (end 142.24 76.2) (width 0.5) (layer B.Cu) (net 6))
 (segment (start 142.24 71.12) (end 142.24 73.66) (width 0.5) (layer B.Cu) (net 6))
 (segment (start 142.24 68.58) (end 142.24 71.12) (width 0.5) (layer B.Cu) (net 6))
 (segment (start 142.24 66.04) (end 142.24 68.58) (width 0.5) (layer B.Cu) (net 6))
 (segment (start 142.24 60.96) (end 142.24 63.5) (width 0.5) (layer B.Cu) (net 6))
 (segment (start 152.4 58.42) (end 153.602081 58.42) (width 0.5) (layer B.Cu) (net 20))
 (segment (start 153.602081 58.42) (end 158.02 58.42) (width 0.5) (layer B.Cu) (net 20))
 (segment (start 152.4 60.96) (end 158.02 60.96) (width 0.5) (layer B.Cu) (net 22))
 (segment (start 152.4 63.5) (end 158.02 63.5) (width 0.5) (layer B.Cu) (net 24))
 (segment (start 152.4 66.04) (end 158.02 66.04) (width 0.5) (layer B.Cu) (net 26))
 (segment (start 152.4 68.58) (end 158.02 68.58) (width 0.5) (layer B.Cu) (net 28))
 (segment (start 152.4 71.12) (end 158.02 71.12) (width 0.5) (layer B.Cu) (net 30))
 (segment (start 152.4 73.66) (end 158.02 73.66) (width 0.5) (layer B.Cu) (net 32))
 (segment (start 152.4 76.2) (end 158.02 76.2) (width 0.5) (layer B.Cu) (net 34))
 (segment (start 144.24 76.2) (end 149.86 76.2) (width 0.5) (layer B.Cu) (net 35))
 (segment (start 144.24 73.66) (end 149.86 73.66) (width 0.5) (layer B.Cu) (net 33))
 (segment (start 144.24 71.12) (end 145.49 71.12) (width 0.5) (layer B.Cu) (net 31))
 (segment (start 145.49 71.12) (end 149.86 71.12) (width 0.5) (layer B.Cu) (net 31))
 (segment (start 144.24 68.58) (end 149.86 68.58) (width 0.5) (layer B.Cu) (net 29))
 (segment (start 144.24 66.04) (end 145.49 66.04) (width 0.5) (layer B.Cu) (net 27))
 (segment (start 145.49 66.04) (end 149.86 66.04) (width 0.5) (layer B.Cu) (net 27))
 (segment (start 144.24 63.5) (end 149.86 63.5) (width 0.5) (layer B.Cu) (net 25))
 (segment (start 144.24 60.96) (end 145.49 60.96) (width 0.5) (layer B.Cu) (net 23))
 (segment (start 145.49 60.96) (end 149.86 60.96) (width 0.5) (layer B.Cu) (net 23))
 (segment (start 144.24 58.42) (end 149.86 58.42) (width 0.5) (layer B.Cu) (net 21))
 (segment (start 143.4 48.5) (end 147.56 48.5) (width 0.5) (layer B.Cu) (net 8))
 (segment (start 147.56 48.5) (end 149.86 50.8) (width 0.5) (layer B.Cu) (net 8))
 (segment (start 142.35 49.5) (end 142.4 49.5) (width 0.5) (layer B.Cu) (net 8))
 (segment (start 142.4 49.5) (end 143.4 48.5) (width 0.5) (layer B.Cu) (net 8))
 (segment (start 140.2 50.6) (end 141.3 49.5) (width 0.5) (layer B.Cu) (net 8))
 (segment (start 141.3 49.5) (end 142.35 49.5) (width 0.5) (layer B.Cu) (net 8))
 (segment (start 138.8 50.6) (end 140.2 50.6) (width 0.5) (layer B.Cu) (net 8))
 (segment (start 137.85 51.6) (end 137.85 51.55) (width 0.5) (layer B.Cu) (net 8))
 (segment (start 137.85 51.55) (end 138.8 50.6) (width 0.5) (layer B.Cu) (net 8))
 (segment (start 158 47.5) (end 153.16 47.5) (width 0.5) (layer B.Cu) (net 8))
 (segment (start 153.16 47.5) (end 152.4 48.26) (width 0.5) (layer B.Cu) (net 8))
 (segment (start 162.2 49.55) (end 159.259998 49.55) (width 0.5) (layer B.Cu) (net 8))
 (segment (start 159.259998 49.55) (end 159 49.290002) (width 0.5) (layer B.Cu) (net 8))
 (segment (start 159 49.290002) (end 159 48.45) (width 0.5) (layer B.Cu) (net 8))
 (segment (start 159 48.45) (end 158.05 47.5) (width 0.5) (layer B.Cu) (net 8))
 (segment (start 158.05 47.5) (end 158 47.5) (width 0.5) (layer B.Cu) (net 8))
 (segment (start 152.4 48.26) (end 149.86 50.8) (width 0.5) (layer B.Cu) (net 8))
 (segment (start 152.4 53.34) (end 153.602081 53.34) (width 0.5) (layer B.Cu) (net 16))
 (segment (start 153.602081 53.34) (end 158.02 53.34) (width 0.5) (layer B.Cu) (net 16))
 (segment (start 144.24 53.34) (end 145.49 53.34) (width 0.5) (layer B.Cu) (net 17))
 (segment (start 145.49 53.34) (end 149.86 53.34) (width 0.5) (layer B.Cu) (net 17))
 (segment (start 152.4 55.88) (end 158.02 55.88) (width 0.5) (layer B.Cu) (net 18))
 (segment (start 144.24 55.88) (end 149.86 55.88) (width 0.5) (layer B.Cu) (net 19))
 (segment (start 139.8 55.9) (end 142.22 55.9) (width 0.5) (layer B.Cu) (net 12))
 (segment (start 142.22 55.9) (end 142.24 55.88) (width 0.5) (layer B.Cu) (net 12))
 (segment (start 142.24 53.34) (end 142.24 51.24) (width 0.5) (layer B.Cu) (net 14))
 (segment (start 142.24 51.24) (end 142.2 51.2) (width 0.5) (layer B.Cu) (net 14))
 (segment (start 160.02 55.88) (end 162.12 55.88) (width 0.5) (layer B.Cu) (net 13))
 (segment (start 162.12 55.88) (end 162.2 55.8) (width 0.5) (layer B.Cu) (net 13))
 (segment (start 160.2 51.3) (end 160.2 53.16) (width 0.5) (layer B.Cu) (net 15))
 (segment (start 160.2 53.16) (end 160.02 53.34) (width 0.5) (layer B.Cu) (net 15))
 (segment (start 139.8 53.7) (end 139.8 51.65) (width 0.5) (layer B.Cu) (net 7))
 (segment (start 139.8 51.65) (end 139.75 51.6) (width 0.5) (layer B.Cu) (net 7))
 (segment (start 162.2 51.45) (end 162.2 53.6) (width 0.5) (layer B.Cu) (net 9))
 (segment (start 144.25 49.5) (end 144.25 51.05) (width 0.5) (layer B.Cu) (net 10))
 (segment (start 144.25 51.05) (end 144.4 51.2) (width 0.5) (layer B.Cu) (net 10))
 (segment (start 158 49.4) (end 158 51.3) (width 0.5) (layer B.Cu) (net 11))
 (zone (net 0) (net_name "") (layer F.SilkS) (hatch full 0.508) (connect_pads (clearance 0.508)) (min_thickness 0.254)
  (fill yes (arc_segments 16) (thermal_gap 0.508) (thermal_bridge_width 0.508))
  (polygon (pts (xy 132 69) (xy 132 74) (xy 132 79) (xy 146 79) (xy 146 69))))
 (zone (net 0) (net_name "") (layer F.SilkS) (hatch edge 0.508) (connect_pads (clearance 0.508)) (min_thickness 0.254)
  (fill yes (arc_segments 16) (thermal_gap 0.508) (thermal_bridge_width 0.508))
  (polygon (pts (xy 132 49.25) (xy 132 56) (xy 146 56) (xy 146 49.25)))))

